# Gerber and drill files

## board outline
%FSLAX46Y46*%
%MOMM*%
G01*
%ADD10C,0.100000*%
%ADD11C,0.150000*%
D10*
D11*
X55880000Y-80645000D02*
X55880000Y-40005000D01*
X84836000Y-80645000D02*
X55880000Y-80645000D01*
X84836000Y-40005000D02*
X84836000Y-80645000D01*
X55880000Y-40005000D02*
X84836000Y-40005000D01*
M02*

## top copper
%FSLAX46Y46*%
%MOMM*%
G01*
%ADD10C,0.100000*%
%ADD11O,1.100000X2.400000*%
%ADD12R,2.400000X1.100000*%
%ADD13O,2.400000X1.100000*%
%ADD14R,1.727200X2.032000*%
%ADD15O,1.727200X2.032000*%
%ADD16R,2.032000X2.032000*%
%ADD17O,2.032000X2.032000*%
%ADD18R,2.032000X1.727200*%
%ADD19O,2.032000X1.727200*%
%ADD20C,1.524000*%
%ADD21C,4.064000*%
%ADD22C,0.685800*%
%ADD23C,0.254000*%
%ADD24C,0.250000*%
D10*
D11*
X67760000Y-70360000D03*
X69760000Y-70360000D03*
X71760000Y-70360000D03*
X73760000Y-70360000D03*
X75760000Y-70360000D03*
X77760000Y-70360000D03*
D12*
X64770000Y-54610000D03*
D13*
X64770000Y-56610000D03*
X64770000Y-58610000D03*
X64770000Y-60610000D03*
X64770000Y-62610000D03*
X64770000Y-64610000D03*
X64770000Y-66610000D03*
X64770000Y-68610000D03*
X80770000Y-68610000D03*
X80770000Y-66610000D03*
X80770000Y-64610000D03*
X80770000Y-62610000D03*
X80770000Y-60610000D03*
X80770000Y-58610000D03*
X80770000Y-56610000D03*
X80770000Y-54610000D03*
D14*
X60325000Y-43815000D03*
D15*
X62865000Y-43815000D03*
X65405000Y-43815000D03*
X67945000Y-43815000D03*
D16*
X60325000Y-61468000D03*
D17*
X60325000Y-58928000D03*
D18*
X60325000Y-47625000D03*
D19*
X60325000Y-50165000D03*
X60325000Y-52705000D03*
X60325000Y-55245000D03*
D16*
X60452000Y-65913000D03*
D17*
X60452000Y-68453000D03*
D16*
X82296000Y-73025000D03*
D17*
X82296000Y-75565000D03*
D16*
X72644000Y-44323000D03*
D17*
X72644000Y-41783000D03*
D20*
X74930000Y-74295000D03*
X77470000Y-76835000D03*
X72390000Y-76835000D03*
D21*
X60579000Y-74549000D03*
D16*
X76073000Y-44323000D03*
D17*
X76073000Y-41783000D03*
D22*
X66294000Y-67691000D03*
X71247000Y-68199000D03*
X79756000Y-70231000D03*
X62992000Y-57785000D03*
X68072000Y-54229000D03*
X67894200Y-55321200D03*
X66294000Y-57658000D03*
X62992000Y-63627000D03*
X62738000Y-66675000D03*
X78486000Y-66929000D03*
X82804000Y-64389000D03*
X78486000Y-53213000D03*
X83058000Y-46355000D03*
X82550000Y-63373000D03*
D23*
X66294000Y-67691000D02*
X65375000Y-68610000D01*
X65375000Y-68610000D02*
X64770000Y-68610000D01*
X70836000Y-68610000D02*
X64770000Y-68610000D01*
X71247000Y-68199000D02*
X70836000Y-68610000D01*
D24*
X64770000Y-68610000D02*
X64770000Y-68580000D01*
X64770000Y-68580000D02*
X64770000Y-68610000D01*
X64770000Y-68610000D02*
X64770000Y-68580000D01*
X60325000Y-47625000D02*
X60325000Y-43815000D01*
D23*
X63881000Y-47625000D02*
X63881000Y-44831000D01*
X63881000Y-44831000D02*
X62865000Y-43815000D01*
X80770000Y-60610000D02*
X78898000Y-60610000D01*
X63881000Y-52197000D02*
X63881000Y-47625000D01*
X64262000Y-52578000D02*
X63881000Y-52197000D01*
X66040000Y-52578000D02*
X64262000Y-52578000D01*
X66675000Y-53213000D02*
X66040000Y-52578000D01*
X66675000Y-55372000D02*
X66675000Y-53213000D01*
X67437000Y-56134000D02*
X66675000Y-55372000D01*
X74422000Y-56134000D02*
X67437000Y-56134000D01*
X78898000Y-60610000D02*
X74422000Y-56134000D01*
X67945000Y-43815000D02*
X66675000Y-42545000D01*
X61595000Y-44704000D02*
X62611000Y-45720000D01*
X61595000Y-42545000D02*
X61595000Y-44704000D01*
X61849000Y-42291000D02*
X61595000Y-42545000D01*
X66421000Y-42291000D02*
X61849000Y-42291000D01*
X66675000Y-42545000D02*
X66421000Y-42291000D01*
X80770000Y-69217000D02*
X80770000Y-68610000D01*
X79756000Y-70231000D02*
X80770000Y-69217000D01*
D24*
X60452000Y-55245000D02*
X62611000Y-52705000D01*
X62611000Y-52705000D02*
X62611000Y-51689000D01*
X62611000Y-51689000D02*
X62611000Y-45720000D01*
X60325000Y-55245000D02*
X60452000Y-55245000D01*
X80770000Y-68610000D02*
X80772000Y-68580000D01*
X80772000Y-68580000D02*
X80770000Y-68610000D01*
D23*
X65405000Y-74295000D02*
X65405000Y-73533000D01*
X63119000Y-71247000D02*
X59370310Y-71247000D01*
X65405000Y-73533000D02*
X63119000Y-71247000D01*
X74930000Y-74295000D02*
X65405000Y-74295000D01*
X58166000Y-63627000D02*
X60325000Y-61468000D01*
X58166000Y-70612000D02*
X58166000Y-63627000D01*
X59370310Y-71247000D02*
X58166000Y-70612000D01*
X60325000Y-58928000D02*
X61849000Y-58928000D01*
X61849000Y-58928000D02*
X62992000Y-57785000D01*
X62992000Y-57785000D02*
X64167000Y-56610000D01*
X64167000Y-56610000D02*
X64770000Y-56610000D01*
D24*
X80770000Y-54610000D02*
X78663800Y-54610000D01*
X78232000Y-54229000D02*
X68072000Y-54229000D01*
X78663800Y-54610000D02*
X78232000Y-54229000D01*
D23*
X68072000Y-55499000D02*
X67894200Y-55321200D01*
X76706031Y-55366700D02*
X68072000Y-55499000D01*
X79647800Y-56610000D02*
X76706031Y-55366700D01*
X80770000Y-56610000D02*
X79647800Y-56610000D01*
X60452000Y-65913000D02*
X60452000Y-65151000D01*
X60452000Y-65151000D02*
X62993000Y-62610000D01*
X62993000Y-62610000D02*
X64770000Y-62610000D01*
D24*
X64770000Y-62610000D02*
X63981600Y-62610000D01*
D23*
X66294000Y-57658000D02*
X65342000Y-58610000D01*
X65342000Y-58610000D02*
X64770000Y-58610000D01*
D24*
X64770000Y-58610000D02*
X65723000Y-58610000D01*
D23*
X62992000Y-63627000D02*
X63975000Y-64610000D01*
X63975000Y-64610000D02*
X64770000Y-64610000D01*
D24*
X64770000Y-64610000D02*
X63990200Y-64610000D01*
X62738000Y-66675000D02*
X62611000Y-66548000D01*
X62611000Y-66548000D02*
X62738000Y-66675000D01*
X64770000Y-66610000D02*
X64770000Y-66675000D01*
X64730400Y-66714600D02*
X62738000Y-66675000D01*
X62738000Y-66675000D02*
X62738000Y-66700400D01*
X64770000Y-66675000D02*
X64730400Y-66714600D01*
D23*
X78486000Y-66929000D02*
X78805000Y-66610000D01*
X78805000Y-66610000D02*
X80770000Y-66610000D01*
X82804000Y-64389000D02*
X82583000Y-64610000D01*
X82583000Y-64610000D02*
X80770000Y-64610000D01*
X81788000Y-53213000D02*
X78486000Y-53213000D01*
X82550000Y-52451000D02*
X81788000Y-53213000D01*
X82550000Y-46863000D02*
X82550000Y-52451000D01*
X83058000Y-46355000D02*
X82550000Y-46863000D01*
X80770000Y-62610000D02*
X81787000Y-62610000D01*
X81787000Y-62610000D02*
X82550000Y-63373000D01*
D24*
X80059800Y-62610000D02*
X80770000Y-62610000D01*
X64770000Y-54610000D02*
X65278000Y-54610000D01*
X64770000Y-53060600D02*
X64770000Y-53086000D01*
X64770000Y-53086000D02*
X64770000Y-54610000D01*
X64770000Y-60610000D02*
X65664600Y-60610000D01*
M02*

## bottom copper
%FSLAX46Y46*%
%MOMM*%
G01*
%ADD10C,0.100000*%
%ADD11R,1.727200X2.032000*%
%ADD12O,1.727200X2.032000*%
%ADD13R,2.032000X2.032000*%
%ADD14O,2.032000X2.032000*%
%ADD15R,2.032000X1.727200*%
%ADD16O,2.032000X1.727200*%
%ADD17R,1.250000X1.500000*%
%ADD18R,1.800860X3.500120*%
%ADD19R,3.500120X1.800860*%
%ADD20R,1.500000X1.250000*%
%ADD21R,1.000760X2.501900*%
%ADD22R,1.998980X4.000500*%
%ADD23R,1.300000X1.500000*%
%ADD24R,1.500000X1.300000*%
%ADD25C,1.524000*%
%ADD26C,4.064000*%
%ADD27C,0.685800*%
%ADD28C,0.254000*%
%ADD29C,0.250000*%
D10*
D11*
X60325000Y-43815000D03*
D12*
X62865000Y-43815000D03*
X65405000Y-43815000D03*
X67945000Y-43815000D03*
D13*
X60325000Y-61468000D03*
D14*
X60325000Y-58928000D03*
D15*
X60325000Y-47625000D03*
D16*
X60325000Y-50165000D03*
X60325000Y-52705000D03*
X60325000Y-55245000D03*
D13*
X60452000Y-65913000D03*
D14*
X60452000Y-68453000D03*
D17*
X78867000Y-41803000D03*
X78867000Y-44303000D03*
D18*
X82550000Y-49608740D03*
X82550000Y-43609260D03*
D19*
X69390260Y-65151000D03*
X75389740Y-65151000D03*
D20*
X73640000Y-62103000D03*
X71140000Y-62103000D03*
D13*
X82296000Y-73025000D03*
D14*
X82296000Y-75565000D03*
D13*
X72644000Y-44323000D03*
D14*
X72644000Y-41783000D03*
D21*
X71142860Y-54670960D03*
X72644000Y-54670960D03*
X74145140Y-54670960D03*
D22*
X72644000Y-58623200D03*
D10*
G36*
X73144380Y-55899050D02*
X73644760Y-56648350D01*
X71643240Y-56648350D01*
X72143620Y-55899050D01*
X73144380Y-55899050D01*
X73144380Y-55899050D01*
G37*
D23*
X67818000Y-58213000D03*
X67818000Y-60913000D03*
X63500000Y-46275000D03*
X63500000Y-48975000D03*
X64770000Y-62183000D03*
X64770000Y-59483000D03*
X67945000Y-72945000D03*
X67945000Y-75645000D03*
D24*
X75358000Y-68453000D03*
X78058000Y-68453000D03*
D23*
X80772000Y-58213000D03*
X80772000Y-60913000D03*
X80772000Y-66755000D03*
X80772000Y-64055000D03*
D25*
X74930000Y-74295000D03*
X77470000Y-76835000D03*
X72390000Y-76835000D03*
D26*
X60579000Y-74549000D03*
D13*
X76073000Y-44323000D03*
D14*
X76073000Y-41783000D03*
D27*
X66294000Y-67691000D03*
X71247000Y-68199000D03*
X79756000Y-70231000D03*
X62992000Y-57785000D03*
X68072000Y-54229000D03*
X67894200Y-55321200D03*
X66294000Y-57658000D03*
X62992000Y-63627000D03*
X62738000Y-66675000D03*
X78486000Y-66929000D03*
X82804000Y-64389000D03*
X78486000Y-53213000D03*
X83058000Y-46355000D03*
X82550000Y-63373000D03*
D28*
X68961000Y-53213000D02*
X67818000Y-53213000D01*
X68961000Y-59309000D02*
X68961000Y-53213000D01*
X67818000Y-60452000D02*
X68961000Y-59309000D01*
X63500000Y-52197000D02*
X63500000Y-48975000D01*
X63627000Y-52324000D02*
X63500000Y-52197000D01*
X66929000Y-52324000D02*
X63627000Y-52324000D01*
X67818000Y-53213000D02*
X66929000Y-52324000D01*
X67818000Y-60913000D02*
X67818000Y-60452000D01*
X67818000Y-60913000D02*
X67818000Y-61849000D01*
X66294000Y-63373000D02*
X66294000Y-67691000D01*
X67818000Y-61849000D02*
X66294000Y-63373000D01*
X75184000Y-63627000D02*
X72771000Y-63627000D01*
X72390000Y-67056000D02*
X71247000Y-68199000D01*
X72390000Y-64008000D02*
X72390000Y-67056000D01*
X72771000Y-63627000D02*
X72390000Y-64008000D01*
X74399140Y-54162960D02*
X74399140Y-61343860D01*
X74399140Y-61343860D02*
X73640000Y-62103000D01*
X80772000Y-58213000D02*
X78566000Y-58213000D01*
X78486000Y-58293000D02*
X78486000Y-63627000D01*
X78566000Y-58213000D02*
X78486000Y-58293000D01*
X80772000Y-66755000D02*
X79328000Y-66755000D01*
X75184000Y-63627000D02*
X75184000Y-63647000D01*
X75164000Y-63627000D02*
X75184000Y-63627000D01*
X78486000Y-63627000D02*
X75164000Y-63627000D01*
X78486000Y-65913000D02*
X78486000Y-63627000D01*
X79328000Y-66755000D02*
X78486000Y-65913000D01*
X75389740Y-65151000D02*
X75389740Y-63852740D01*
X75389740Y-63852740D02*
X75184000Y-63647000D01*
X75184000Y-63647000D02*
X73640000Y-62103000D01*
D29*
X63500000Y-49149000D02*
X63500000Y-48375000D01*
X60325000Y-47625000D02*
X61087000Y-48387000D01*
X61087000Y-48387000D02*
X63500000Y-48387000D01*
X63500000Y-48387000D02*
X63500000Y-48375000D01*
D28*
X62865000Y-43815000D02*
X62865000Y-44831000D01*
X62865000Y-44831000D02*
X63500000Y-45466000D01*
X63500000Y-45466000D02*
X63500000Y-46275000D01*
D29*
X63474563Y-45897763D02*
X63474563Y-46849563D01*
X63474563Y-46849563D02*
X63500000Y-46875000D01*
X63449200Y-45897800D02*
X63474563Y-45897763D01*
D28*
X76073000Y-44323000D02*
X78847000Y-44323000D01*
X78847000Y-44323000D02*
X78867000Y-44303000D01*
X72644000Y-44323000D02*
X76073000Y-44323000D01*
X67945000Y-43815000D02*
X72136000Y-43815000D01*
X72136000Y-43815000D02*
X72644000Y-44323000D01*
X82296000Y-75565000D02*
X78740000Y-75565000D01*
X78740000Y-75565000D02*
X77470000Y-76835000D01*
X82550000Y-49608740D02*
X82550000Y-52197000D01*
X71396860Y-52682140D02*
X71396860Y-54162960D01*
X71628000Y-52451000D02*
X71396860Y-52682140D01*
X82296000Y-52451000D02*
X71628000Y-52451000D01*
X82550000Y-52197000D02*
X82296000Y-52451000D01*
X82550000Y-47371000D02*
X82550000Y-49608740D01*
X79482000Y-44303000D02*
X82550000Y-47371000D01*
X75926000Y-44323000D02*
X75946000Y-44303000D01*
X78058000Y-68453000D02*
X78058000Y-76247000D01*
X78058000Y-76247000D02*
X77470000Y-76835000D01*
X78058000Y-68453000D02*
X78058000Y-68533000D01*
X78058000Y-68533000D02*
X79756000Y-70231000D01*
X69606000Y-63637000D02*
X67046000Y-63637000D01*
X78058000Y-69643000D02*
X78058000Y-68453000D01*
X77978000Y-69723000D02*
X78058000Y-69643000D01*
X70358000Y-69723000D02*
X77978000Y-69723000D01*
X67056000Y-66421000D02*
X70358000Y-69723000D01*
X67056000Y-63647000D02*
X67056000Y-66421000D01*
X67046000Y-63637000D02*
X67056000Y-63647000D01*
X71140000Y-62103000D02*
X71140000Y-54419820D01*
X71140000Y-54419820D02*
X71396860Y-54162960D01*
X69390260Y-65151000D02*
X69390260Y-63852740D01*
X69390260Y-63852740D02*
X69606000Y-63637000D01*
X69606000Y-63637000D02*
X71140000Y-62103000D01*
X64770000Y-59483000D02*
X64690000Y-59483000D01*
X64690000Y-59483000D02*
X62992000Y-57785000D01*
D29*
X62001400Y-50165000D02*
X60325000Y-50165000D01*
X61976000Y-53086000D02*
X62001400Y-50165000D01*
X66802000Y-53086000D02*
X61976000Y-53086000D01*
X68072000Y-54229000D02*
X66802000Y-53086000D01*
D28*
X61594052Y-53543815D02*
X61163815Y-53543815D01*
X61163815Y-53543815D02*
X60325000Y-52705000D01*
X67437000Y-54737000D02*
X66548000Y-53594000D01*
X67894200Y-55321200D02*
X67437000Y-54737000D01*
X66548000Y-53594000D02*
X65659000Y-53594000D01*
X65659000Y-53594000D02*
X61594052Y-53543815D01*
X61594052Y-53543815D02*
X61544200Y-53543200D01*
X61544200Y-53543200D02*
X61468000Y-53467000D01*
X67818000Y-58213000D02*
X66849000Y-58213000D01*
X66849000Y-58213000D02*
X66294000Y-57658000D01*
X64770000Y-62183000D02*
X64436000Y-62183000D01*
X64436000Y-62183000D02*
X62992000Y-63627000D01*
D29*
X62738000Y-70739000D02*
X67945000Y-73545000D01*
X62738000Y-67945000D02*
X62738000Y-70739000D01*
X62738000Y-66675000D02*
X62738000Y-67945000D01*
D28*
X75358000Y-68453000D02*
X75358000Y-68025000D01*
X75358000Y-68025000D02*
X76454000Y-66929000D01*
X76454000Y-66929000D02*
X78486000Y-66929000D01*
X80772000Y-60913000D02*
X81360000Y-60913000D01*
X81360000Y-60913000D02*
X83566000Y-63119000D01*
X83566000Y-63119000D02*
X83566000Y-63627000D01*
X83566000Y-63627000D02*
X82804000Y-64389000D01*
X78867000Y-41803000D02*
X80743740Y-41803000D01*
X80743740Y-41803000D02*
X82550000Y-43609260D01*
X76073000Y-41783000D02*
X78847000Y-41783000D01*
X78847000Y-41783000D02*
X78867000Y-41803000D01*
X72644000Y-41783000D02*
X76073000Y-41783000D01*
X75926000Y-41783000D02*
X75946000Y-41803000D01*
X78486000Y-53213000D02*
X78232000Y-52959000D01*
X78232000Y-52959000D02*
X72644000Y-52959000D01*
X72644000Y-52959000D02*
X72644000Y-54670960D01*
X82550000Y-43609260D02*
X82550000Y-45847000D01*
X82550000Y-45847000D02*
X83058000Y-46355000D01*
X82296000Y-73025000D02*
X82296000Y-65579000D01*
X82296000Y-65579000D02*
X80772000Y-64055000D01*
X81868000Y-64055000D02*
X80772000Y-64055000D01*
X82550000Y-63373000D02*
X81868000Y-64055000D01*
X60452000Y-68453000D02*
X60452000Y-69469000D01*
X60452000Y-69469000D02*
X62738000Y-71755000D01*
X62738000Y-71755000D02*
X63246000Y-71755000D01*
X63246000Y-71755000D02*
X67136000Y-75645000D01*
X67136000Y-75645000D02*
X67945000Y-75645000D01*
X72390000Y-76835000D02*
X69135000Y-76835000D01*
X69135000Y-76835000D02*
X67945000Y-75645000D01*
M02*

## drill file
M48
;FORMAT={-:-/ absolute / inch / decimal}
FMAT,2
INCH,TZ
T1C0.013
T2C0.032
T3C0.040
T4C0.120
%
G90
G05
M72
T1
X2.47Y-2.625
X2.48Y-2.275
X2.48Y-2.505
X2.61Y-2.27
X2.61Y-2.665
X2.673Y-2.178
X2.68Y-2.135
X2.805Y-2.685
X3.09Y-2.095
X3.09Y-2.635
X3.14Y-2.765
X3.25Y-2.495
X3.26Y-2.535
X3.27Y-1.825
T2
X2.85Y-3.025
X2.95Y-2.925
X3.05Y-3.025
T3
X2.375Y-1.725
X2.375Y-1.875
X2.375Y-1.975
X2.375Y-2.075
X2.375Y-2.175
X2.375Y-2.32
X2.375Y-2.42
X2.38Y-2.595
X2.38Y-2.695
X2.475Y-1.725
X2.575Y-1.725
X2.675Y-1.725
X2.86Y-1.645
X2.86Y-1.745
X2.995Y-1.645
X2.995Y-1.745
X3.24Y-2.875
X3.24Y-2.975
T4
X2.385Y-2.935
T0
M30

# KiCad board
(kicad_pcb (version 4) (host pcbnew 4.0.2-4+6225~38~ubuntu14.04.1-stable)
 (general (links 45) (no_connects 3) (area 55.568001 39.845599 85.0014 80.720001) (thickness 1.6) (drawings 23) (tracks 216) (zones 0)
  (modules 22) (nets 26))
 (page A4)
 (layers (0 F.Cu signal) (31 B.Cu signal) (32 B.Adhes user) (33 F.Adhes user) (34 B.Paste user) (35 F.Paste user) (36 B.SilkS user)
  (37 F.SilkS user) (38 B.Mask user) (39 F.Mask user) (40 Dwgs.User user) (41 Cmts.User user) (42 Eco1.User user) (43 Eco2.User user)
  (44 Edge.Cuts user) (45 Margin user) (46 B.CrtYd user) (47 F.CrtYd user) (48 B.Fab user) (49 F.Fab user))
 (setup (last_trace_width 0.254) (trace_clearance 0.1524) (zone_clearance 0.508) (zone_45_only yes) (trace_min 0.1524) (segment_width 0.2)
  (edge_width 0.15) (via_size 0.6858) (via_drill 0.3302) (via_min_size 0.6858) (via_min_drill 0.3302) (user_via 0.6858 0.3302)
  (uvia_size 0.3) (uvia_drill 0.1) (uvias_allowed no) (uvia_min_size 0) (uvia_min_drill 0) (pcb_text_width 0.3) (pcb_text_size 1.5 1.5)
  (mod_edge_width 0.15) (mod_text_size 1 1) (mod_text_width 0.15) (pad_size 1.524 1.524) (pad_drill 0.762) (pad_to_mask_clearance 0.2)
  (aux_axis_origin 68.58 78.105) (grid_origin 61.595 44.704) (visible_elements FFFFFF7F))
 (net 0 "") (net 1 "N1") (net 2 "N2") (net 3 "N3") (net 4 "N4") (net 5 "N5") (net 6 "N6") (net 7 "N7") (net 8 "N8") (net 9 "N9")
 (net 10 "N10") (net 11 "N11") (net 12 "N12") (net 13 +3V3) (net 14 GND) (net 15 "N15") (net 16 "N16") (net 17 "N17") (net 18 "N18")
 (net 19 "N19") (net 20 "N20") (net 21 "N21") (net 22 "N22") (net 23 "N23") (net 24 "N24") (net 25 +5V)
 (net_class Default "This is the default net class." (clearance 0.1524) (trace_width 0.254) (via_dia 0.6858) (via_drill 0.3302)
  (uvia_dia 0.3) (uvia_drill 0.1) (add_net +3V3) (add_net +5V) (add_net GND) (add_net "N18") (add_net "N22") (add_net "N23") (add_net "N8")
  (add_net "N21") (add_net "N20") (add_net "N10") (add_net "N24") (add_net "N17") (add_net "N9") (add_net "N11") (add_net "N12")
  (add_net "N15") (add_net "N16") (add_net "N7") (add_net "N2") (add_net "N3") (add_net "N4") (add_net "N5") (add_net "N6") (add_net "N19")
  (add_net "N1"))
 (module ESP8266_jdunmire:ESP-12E (layer F.Cu) (at 64.77 54.61)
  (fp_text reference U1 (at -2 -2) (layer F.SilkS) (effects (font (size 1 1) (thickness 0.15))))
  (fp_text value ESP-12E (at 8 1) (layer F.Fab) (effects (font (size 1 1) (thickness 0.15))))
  (pad 9 smd oval (at 2.99 15.75 90) (size 2.4 1.1) (layers F.Cu F.Paste F.Mask) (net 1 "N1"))
  (pad 10 smd oval (at 4.99 15.75 90) (size 2.4 1.1) (layers F.Cu F.Paste F.Mask) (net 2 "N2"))
  (pad 11 smd oval (at 6.99 15.75 90) (size 2.4 1.1) (layers F.Cu F.Paste F.Mask) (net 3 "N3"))
  (pad 12 smd oval (at 8.99 15.75 90) (size 2.4 1.1) (layers F.Cu F.Paste F.Mask) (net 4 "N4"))
  (pad 13 smd oval (at 10.99 15.75 90) (size 2.4 1.1) (layers F.Cu F.Paste F.Mask) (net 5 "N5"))
  (pad 14 smd oval (at 12.99 15.75 90) (size 2.4 1.1) (layers F.Cu F.Paste F.Mask) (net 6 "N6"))
  (pad 1 smd rect (at 0 0) (size 2.4 1.1) (layers F.Cu F.Paste F.Mask) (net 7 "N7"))
  (pad 2 smd oval (at 0 2) (size 2.4 1.1) (layers F.Cu F.Paste F.Mask) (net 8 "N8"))
  (pad 3 smd oval (at 0 4) (size 2.4 1.1) (layers F.Cu F.Paste F.Mask) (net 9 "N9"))
  (pad 4 smd oval (at 0 6) (size 2.4 1.1) (layers F.Cu F.Paste F.Mask) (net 7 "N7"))
  (pad 5 smd oval (at 0 8) (size 2.4 1.1) (layers F.Cu F.Paste F.Mask) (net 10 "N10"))
  (pad 6 smd oval (at 0 10) (size 2.4 1.1) (layers F.Cu F.Paste F.Mask) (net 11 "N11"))
  (pad 7 smd oval (at 0 12) (size 2.4 1.1) (layers F.Cu F.Paste F.Mask) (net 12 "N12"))
  (pad 8 smd oval (at 0 14) (size 2.4 1.1) (layers F.Cu F.Paste F.Mask) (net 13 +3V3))
  (pad 15 smd oval (at 16 14) (size 2.4 1.1) (layers F.Cu F.Paste F.Mask) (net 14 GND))
  (pad 16 smd oval (at 16 12) (size 2.4 1.1) (layers F.Cu F.Paste F.Mask) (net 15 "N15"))
  (pad 17 smd oval (at 16 10) (size 2.4 1.1) (layers F.Cu F.Paste F.Mask) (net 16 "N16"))
  (pad 18 smd oval (at 16 8) (size 2.4 1.1) (layers F.Cu F.Paste F.Mask) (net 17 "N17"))
  (pad 19 smd oval (at 16 6) (size 2.4 1.1) (layers F.Cu F.Paste F.Mask) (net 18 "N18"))
  (pad 20 smd oval (at 16 4) (size 2.4 1.1) (layers F.Cu F.Paste F.Mask) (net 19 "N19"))
  (pad 21 smd oval (at 16 2) (size 2.4 1.1) (layers F.Cu F.Paste F.Mask) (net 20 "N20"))
  (pad 22 smd oval (at 16 0) (size 2.4 1.1) (layers F.Cu F.Paste F.Mask) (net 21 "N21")))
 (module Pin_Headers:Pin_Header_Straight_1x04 (layer F.Cu) (at 60.325 43.815 90)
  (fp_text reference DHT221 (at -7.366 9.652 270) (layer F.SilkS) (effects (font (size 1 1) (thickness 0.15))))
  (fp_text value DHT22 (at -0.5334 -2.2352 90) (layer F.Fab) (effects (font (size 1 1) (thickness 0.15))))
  (pad 1 thru_hole rect (at 0 0 90) (size 2.032 1.7272) (drill 1.016) (layers *.Cu *.Mask F.SilkS) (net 13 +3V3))
  (pad 2 thru_hole oval (at 0 2.54 90) (size 2.032 1.7272) (drill 1.016) (layers *.Cu *.Mask F.SilkS) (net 18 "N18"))
  (pad 3 thru_hole oval (at 0 5.08 90) (size 2.032 1.7272) (drill 1.016) (layers *.Cu *.Mask F.SilkS) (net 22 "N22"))
  (pad 4 thru_hole oval (at 0 7.62 90) (size 2.032 1.7272) (drill 1.016) (layers *.Cu *.Mask F.SilkS) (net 14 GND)))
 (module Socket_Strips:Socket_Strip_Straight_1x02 (layer F.Cu) (at 60.325 61.468 90)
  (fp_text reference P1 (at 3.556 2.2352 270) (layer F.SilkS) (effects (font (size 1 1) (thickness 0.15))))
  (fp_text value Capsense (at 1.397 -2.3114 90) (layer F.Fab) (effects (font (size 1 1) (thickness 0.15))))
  (pad 1 thru_hole rect (at 0 0 90) (size 2.032 2.032) (drill 1.016) (layers *.Cu *.Mask F.SilkS) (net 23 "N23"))
  (pad 2 thru_hole oval (at 2.54 0 90) (size 2.032 2.032) (drill 1.016) (layers *.Cu *.Mask F.SilkS) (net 8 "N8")))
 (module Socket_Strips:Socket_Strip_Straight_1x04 (layer F.Cu) (at 60.325 47.625 270)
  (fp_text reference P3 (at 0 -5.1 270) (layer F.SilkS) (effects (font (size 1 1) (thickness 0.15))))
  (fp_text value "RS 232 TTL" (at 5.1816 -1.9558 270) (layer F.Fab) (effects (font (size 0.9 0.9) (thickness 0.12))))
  (pad 1 thru_hole rect (at 0 0 270) (size 1.7272 2.032) (drill 1.016) (layers *.Cu *.Mask F.SilkS) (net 13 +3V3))
  (pad 2 thru_hole oval (at 2.54 0 270) (size 1.7272 2.032) (drill 1.016) (layers *.Cu *.Mask F.SilkS) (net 21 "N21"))
  (pad 3 thru_hole oval (at 5.08 0 270) (size 1.7272 2.032) (drill 1.016) (layers *.Cu *.Mask F.SilkS) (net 20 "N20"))
  (pad 4 thru_hole oval (at 7.62 0 270) (size 1.7272 2.032) (drill 1.016) (layers *.Cu *.Mask F.SilkS) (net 14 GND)))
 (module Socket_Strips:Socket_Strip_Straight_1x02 (layer F.Cu) (at 60.452 65.913 270)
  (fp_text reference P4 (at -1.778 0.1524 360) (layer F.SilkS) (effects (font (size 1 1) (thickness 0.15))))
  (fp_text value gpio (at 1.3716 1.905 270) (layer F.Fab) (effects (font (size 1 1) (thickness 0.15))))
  (pad 1 thru_hole rect (at 0 0 270) (size 2.032 2.032) (drill 1.016) (layers *.Cu *.Mask F.SilkS) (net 10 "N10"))
  (pad 2 thru_hole oval (at 2.54 0 270) (size 2.032 2.032) (drill 1.016) (layers *.Cu *.Mask F.SilkS) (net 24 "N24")))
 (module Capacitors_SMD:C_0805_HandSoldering (layer B.Cu) (at 78.867 43.053 270)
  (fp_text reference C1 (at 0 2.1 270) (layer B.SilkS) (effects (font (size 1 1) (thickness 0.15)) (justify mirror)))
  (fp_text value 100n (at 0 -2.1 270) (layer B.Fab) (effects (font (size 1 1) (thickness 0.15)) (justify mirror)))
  (pad 1 smd rect (at -1.25 0 270) (size 1.5 1.25) (layers B.Cu B.Paste B.Mask) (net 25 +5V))
  (pad 2 smd rect (at 1.25 0 270) (size 1.5 1.25) (layers B.Cu B.Paste B.Mask) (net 14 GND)))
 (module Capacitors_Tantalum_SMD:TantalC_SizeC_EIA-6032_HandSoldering (layer B.Cu) (at 82.55 46.609 270)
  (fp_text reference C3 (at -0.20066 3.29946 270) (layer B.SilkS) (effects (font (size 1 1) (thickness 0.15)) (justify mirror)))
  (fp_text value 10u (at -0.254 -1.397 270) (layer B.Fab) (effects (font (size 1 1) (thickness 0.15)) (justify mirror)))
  (pad 2 smd rect (at 2.99974 0 270) (size 3.50012 1.80086) (layers B.Cu B.Paste B.Mask) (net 14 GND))
  (pad 1 smd rect (at -2.99974 0 270) (size 3.50012 1.80086) (layers B.Cu B.Paste B.Mask) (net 25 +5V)))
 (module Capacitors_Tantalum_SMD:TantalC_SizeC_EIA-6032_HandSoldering (layer B.Cu) (at 72.39 65.151 180)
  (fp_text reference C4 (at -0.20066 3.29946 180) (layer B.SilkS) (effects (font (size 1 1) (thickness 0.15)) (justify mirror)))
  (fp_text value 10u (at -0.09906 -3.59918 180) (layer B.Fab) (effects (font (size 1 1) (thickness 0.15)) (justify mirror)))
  (pad 2 smd rect (at 2.99974 0 180) (size 3.50012 1.80086) (layers B.Cu B.Paste B.Mask) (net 14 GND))
  (pad 1 smd rect (at -2.99974 0 180) (size 3.50012 1.80086) (layers B.Cu B.Paste B.Mask) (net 13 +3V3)))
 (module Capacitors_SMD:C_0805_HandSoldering (layer B.Cu) (at 72.39 62.103 180)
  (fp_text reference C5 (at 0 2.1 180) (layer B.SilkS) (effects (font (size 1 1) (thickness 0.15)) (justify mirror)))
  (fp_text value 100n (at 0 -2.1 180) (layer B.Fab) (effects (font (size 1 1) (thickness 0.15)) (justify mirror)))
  (pad 1 smd rect (at -1.25 0 180) (size 1.5 1.25) (layers B.Cu B.Paste B.Mask) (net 13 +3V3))
  (pad 2 smd rect (at 1.25 0 180) (size 1.5 1.25) (layers B.Cu B.Paste B.Mask) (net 14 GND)))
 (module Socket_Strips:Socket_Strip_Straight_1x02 (layer F.Cu) (at 82.296 73.025 270)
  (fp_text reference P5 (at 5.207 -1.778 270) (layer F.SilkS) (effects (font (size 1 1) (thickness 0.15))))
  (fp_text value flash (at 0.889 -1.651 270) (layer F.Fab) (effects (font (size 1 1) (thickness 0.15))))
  (pad 1 thru_hole rect (at 0 0 270) (size 2.032 2.032) (drill 1.016) (layers *.Cu *.Mask F.SilkS) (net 17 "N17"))
  (pad 2 thru_hole oval (at 2.54 0 270) (size 2.032 2.032) (drill 1.016) (layers *.Cu *.Mask F.SilkS) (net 14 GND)))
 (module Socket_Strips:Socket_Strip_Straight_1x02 (layer F.Cu) (at 72.644 44.323 90)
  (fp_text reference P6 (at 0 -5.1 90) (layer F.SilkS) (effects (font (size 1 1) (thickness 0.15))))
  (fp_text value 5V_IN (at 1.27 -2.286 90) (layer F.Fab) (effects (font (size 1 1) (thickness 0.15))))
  (pad 1 thru_hole rect (at 0 0 90) (size 2.032 2.032) (drill 1.016) (layers *.Cu *.Mask F.SilkS) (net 14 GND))
  (pad 2 thru_hole oval (at 2.54 0 90) (size 2.032 2.032) (drill 1.016) (layers *.Cu *.Mask F.SilkS) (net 25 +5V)))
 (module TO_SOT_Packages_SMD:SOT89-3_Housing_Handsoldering (layer B.Cu) (at 72.644 57.023)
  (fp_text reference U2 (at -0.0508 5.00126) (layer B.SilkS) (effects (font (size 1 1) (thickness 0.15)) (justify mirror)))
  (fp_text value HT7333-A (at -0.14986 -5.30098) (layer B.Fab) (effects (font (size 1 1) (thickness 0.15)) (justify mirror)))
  (pad 1 smd rect (at -1.50114 -2.35204) (size 1.00076 2.5019) (layers B.Cu B.Paste B.Mask) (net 14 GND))
  (pad 2 smd rect (at 0 -2.35204) (size 1.00076 2.5019) (layers B.Cu B.Paste B.Mask) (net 25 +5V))
  (pad 3 smd rect (at 1.50114 -2.35204) (size 1.00076 2.5019) (layers B.Cu B.Paste B.Mask) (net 13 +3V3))
  (pad 2 smd rect (at 0 1.6002) (size 1.99898 4.0005) (layers B.Cu B.Paste B.Mask) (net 25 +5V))
  (pad 2 smd trapezoid (at 0 -0.7493 180) (size 1.50114 0.7493) (rect_delta 0 -0.50038) (layers B.Cu B.Paste B.Mask) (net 25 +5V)))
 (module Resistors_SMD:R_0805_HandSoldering (layer B.Cu) (at 67.818 59.563 270)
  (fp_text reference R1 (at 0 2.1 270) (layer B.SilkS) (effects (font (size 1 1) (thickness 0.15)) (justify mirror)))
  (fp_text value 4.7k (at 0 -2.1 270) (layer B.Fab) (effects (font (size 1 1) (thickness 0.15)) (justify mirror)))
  (pad 1 smd rect (at -1.35 0 270) (size 1.5 1.3) (layers B.Cu B.Paste B.Mask) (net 9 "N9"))
  (pad 2 smd rect (at 1.35 0 270) (size 1.5 1.3) (layers B.Cu B.Paste B.Mask) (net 13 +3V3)))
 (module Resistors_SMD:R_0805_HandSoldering (layer B.Cu) (at 63.5 47.625 270)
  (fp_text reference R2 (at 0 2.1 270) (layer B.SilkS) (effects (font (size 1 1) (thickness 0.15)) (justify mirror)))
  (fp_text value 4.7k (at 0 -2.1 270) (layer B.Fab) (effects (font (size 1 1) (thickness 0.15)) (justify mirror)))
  (pad 1 smd rect (at -1.35 0 270) (size 1.5 1.3) (layers B.Cu B.Paste B.Mask) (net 18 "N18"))
  (pad 2 smd rect (at 1.35 0 270) (size 1.5 1.3) (layers B.Cu B.Paste B.Mask) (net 13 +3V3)))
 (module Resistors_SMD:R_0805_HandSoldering (layer B.Cu) (at 64.77 60.833 90)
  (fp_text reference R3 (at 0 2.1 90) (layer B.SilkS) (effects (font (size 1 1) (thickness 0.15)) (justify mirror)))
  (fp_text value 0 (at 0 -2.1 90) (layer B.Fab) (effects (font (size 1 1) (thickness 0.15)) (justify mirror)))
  (pad 1 smd rect (at -1.35 0 90) (size 1.5 1.3) (layers B.Cu B.Paste B.Mask) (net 11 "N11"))
  (pad 2 smd rect (at 1.35 0 90) (size 1.5 1.3) (layers B.Cu B.Paste B.Mask) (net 8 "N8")))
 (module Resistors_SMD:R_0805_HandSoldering (layer B.Cu) (at 67.945 74.295 270)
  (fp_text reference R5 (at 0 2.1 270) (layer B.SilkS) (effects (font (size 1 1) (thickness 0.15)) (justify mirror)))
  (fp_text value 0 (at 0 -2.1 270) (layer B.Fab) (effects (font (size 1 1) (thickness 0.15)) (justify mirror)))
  (pad 1 smd rect (at -1.35 0 270) (size 1.5 1.3) (layers B.Cu B.Paste B.Mask) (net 12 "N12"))
  (pad 2 smd rect (at 1.35 0 270) (size 1.5 1.3) (layers B.Cu B.Paste B.Mask) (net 24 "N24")))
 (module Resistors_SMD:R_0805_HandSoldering (layer B.Cu) (at 76.708 68.453)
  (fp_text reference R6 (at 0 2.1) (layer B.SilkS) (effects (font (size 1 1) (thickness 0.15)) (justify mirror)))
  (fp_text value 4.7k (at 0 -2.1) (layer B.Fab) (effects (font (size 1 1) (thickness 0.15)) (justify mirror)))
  (pad 1 smd rect (at -1.35 0) (size 1.5 1.3) (layers B.Cu B.Paste B.Mask) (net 15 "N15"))
  (pad 2 smd rect (at 1.35 0) (size 1.5 1.3) (layers B.Cu B.Paste B.Mask) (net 14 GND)))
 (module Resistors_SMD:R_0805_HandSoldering (layer B.Cu) (at 80.772 59.563 270)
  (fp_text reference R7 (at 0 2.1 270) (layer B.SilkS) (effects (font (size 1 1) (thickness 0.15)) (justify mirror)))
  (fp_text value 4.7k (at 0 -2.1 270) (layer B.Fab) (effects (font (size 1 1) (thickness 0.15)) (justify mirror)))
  (pad 1 smd rect (at -1.35 0 270) (size 1.5 1.3) (layers B.Cu B.Paste B.Mask) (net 13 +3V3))
  (pad 2 smd rect (at 1.35 0 270) (size 1.5 1.3) (layers B.Cu B.Paste B.Mask) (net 16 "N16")))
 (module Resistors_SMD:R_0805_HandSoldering (layer B.Cu) (at 80.772 65.405 90)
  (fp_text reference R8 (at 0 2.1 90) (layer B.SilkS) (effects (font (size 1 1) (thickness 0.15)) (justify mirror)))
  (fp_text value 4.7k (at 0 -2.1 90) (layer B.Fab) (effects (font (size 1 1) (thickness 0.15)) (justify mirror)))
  (pad 1 smd rect (at -1.35 0 90) (size 1.5 1.3) (layers B.Cu B.Paste B.Mask) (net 13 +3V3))
  (pad 2 smd rect (at 1.35 0 90) (size 1.5 1.3) (layers B.Cu B.Paste B.Mask) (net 17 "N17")))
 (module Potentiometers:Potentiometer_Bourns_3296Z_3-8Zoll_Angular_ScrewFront (layer F.Cu) (at 72.39 76.835 270)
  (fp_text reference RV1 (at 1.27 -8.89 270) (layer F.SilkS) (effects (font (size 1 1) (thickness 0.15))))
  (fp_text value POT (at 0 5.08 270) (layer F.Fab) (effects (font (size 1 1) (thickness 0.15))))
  (pad 2 thru_hole circle (at -2.54 -2.54 270) (size 1.524 1.524) (drill 0.8128) (layers *.Cu *.Mask F.SilkS) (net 23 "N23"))
  (pad 3 thru_hole circle (at 0 -5.08 270) (size 1.524 1.524) (drill 0.8128) (layers *.Cu *.Mask F.SilkS) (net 14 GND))
  (pad 1 thru_hole circle (at 0 0 270) (size 1.524 1.524) (drill 0.8128) (layers *.Cu *.Mask F.SilkS) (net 24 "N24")))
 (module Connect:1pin (layer F.Cu) (at 60.579 74.549)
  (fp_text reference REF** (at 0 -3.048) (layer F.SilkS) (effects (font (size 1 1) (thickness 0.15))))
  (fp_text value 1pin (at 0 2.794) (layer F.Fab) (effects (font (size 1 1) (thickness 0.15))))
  (pad 1 thru_hole circle (at 0 0) (size 4.064 4.064) (drill 3.048) (layers *.Cu *.Mask F.SilkS)))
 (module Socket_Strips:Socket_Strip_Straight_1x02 (layer F.Cu) (at 76.073 44.323 90)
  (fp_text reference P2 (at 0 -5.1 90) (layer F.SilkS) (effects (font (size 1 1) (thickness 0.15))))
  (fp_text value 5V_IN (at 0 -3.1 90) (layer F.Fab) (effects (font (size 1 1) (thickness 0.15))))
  (pad 1 thru_hole rect (at 0 0 90) (size 2.032 2.032) (drill 1.016) (layers *.Cu *.Mask F.SilkS) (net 14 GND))
  (pad 2 thru_hole oval (at 2.54 0 90) (size 2.032 2.032) (drill 1.016) (layers *.Cu *.Mask F.SilkS) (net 25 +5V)))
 (gr_line (start 55.88 80.645) (end 55.88 40.005) (angle 90) (layer Edge.Cuts) (width 0.15))
 (gr_line (start 84.836 80.645) (end 55.88 80.645) (angle 90) (layer Edge.Cuts) (width 0.15))
 (gr_line (start 84.836 40.005) (end 84.836 80.645) (angle 90) (layer Edge.Cuts) (width 0.15))
 (gr_line (start 55.88 40.005) (end 84.836 40.005) (angle 90) (layer Edge.Cuts) (width 0.15))
 (segment (start 68.961 53.213) (end 67.818 53.213) (width 0.254) (layer B.Cu) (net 13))
 (segment (start 68.961 59.309) (end 68.961 53.213) (width 0.254) (layer B.Cu) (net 13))
 (segment (start 67.818 60.452) (end 68.961 59.309) (width 0.254) (layer B.Cu) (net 13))
 (segment (start 63.5 52.197) (end 63.5 48.975) (width 0.254) (layer B.Cu) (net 13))
 (segment (start 63.627 52.324) (end 63.5 52.197) (width 0.254) (layer B.Cu) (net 13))
 (segment (start 66.929 52.324) (end 63.627 52.324) (width 0.254) (layer B.Cu) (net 13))
 (segment (start 67.818 53.213) (end 66.929 52.324) (width 0.254) (layer B.Cu) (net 13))
 (segment (start 67.818 60.913) (end 67.818 60.452) (width 0.254) (layer B.Cu) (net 13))
 (segment (start 67.818 60.913) (end 67.818 61.849) (width 0.254) (layer B.Cu) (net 13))
 (segment (start 66.294 67.691) (end 65.375 68.61) (width 0.254) (layer F.Cu) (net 13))
 (via (at 66.294 67.691) (size 0.6858) (drill 0.3302) (layers F.Cu B.Cu) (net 13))
 (segment (start 66.294 63.373) (end 66.294 67.691) (width 0.254) (layer B.Cu) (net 13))
 (segment (start 67.818 61.849) (end 66.294 63.373) (width 0.254) (layer B.Cu) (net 13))
 (segment (start 65.375 68.61) (end 64.77 68.61) (width 0.254) (layer F.Cu) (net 13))
 (segment (start 75.184 63.627) (end 72.771 63.627) (width 0.254) (layer B.Cu) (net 13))
 (segment (start 70.836 68.61) (end 64.77 68.61) (width 0.254) (layer F.Cu) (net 13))
 (segment (start 71.247 68.199) (end 70.836 68.61) (width 0.254) (layer F.Cu) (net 13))
 (via (at 71.247 68.199) (size 0.6858) (drill 0.3302) (layers F.Cu B.Cu) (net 13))
 (segment (start 72.39 67.056) (end 71.247 68.199) (width 0.254) (layer B.Cu) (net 13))
 (segment (start 72.39 64.008) (end 72.39 67.056) (width 0.254) (layer B.Cu) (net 13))
 (segment (start 72.771 63.627) (end 72.39 64.008) (width 0.254) (layer B.Cu) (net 13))
 (segment (start 74.39914 54.16296) (end 74.39914 61.34386) (width 0.254) (layer B.Cu) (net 13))
 (segment (start 74.39914 61.34386) (end 73.64 62.103) (width 0.254) (layer B.Cu) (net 13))
 (segment (start 80.772 58.213) (end 78.566 58.213) (width 0.254) (layer B.Cu) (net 13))
 (segment (start 78.486 58.293) (end 78.486 63.627) (width 0.254) (layer B.Cu) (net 13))
 (segment (start 78.566 58.213) (end 78.486 58.293) (width 0.254) (layer B.Cu) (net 13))
 (segment (start 80.772 66.755) (end 79.328 66.755) (width 0.254) (layer B.Cu) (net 13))
 (segment (start 75.184 63.627) (end 75.184 63.647) (width 0.254) (layer B.Cu) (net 13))
 (segment (start 75.164 63.627) (end 75.184 63.627) (width 0.254) (layer B.Cu) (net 13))
 (segment (start 78.486 63.627) (end 75.164 63.627) (width 0.254) (layer B.Cu) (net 13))
 (segment (start 78.486 65.913) (end 78.486 63.627) (width 0.254) (layer B.Cu) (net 13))
 (segment (start 79.328 66.755) (end 78.486 65.913) (width 0.254) (layer B.Cu) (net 13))
 (segment (start 75.38974 65.151) (end 75.38974 63.85274) (width 0.254) (layer B.Cu) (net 13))
 (segment (start 75.38974 63.85274) (end 75.184 63.647) (width 0.254) (layer B.Cu) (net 13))
 (segment (start 75.184 63.647) (end 73.64 62.103) (width 0.254) (layer B.Cu) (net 13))
 (segment (start 63.5 49.149) (end 63.5 48.375) (width 0.25) (layer B.Cu) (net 13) (status 80000))
 (segment (start 64.77 68.61) (end 64.77 68.58) (width 0.25) (layer F.Cu) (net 13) (status 80000))
 (segment (start 64.77 68.58) (end 64.77 68.61) (width 0.25) (layer F.Cu) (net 13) (status 80000))
 (segment (start 64.77 68.61) (end 64.77 68.58) (width 0.25) (layer F.Cu) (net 13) (status 80000))
 (segment (start 60.325 47.625) (end 61.087 48.387) (width 0.25) (layer B.Cu) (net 13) (status 80000))
 (segment (start 61.087 48.387) (end 63.5 48.387) (width 0.25) (layer B.Cu) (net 13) (status 80000))
 (segment (start 63.5 48.387) (end 63.5 48.375) (width 0.25) (layer B.Cu) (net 13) (status 80000))
 (segment (start 60.325 47.625) (end 60.325 43.815) (width 0.25) (layer F.Cu) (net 13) (status 80000))
 (segment (start 62.865 43.815) (end 62.865 44.831) (width 0.254) (layer B.Cu) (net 18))
 (segment (start 62.865 44.831) (end 63.5 45.466) (width 0.254) (layer B.Cu) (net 18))
 (segment (start 63.5 45.466) (end 63.5 46.275) (width 0.254) (layer B.Cu) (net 18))
 (segment (start 63.881 47.625) (end 63.881 44.831) (width 0.254) (layer F.Cu) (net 18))
 (segment (start 63.881 44.831) (end 62.865 43.815) (width 0.254) (layer F.Cu) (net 18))
 (segment (start 80.77 60.61) (end 78.898 60.61) (width 0.254) (layer F.Cu) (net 18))
 (segment (start 63.881 52.197) (end 63.881 47.625) (width 0.254) (layer F.Cu) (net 18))
 (segment (start 64.262 52.578) (end 63.881 52.197) (width 0.254) (layer F.Cu) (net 18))
 (segment (start 66.04 52.578) (end 64.262 52.578) (width 0.254) (layer F.Cu) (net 18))
 (segment (start 66.675 53.213) (end 66.04 52.578) (width 0.254) (layer F.Cu) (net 18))
 (segment (start 66.675 55.372) (end 66.675 53.213) (width 0.254) (layer F.Cu) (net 18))
 (segment (start 67.437 56.134) (end 66.675 55.372) (width 0.254) (layer F.Cu) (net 18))
 (segment (start 74.422 56.134) (end 67.437 56.134) (width 0.254) (layer F.Cu) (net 18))
 (segment (start 78.898 60.61) (end 74.422 56.134) (width 0.254) (layer F.Cu) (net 18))
 (segment (start 63.474563 45.897763) (end 63.474563 46.849563) (width 0.25) (layer B.Cu) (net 18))
 (segment (start 63.474563 46.849563) (end 63.5 46.875) (width 0.25) (layer B.Cu) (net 18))
 (segment (start 63.4492 45.8978) (end 63.474563 45.897763) (width 0.25) (layer B.Cu) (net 18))
 (segment (start 76.073 44.323) (end 78.847 44.323) (width 0.254) (layer B.Cu) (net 14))
 (segment (start 78.847 44.323) (end 78.867 44.303) (width 0.254) (layer B.Cu) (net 14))
 (segment (start 72.644 44.323) (end 76.073 44.323) (width 0.254) (layer B.Cu) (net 14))
 (segment (start 67.945 43.815) (end 66.675 42.545) (width 0.254) (layer F.Cu) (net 14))
 (segment (start 61.595 44.704) (end 62.611 45.72) (width 0.254) (layer F.Cu) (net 14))
 (segment (start 61.595 42.545) (end 61.595 44.704) (width 0.254) (layer F.Cu) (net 14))
 (segment (start 61.849 42.291) (end 61.595 42.545) (width 0.254) (layer F.Cu) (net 14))
 (segment (start 66.421 42.291) (end 61.849 42.291) (width 0.254) (layer F.Cu) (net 14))
 (segment (start 66.675 42.545) (end 66.421 42.291) (width 0.254) (layer F.Cu) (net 14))
 (segment (start 67.945 43.815) (end 72.136 43.815) (width 0.254) (layer B.Cu) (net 14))
 (segment (start 72.136 43.815) (end 72.644 44.323) (width 0.254) (layer B.Cu) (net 14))
 (segment (start 82.296 75.565) (end 78.74 75.565) (width 0.254) (layer B.Cu) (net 14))
 (segment (start 78.74 75.565) (end 77.47 76.835) (width 0.254) (layer B.Cu) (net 14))
 (segment (start 82.55 49.60874) (end 82.55 52.197) (width 0.254) (layer B.Cu) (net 14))
 (segment (start 71.39686 52.68214) (end 71.39686 54.16296) (width 0.254) (layer B.Cu) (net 14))
 (segment (start 71.628 52.451) (end 71.39686 52.68214) (width 0.254) (layer B.Cu) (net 14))
 (segment (start 82.296 52.451) (end 71.628 52.451) (width 0.254) (layer B.Cu) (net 14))
 (segment (start 82.55 52.197) (end 82.296 52.451) (width 0.254) (layer B.Cu) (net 14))
 (segment (start 82.55 47.371) (end 82.55 49.60874) (width 0.254) (layer B.Cu) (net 14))
 (segment (start 79.482 44.303) (end 82.55 47.371) (width 0.254) (layer B.Cu) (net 14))
 (segment (start 75.926 44.323) (end 75.946 44.303) (width 0.254) (layer B.Cu) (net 14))
 (segment (start 78.058 68.453) (end 78.058 76.247) (width 0.254) (layer B.Cu) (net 14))
 (segment (start 78.058 76.247) (end 77.47 76.835) (width 0.254) (layer B.Cu) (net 14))
 (segment (start 78.058 68.453) (end 78.058 68.533) (width 0.254) (layer B.Cu) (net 14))
 (segment (start 78.058 68.533) (end 79.756 70.231) (width 0.254) (layer B.Cu) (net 14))
 (segment (start 80.77 69.217) (end 80.77 68.61) (width 0.254) (layer F.Cu) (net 14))
 (segment (start 79.756 70.231) (end 80.77 69.217) (width 0.254) (layer F.Cu) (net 14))
 (via (at 79.756 70.231) (size 0.6858) (drill 0.3302) (layers F.Cu B.Cu) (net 14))
 (segment (start 69.606 63.637) (end 67.046 63.637) (width 0.254) (layer B.Cu) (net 14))
 (segment (start 78.058 69.643) (end 78.058 68.453) (width 0.254) (layer B.Cu) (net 14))
 (segment (start 77.978 69.723) (end 78.058 69.643) (width 0.254) (layer B.Cu) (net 14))
 (segment (start 70.358 69.723) (end 77.978 69.723) (width 0.254) (layer B.Cu) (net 14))
 (segment (start 67.056 66.421) (end 70.358 69.723) (width 0.254) (layer B.Cu) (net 14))
 (segment (start 67.056 63.647) (end 67.056 66.421) (width 0.254) (layer B.Cu) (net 14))
 (segment (start 67.046 63.637) (end 67.056 63.647) (width 0.254) (layer B.Cu) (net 14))
 (segment (start 71.14 62.103) (end 71.14 54.41982) (width 0.254) (layer B.Cu) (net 14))
 (segment (start 71.14 54.41982) (end 71.39686 54.16296) (width 0.254) (layer B.Cu) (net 14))
 (segment (start 69.39026 65.151) (end 69.39026 63.85274) (width 0.254) (layer B.Cu) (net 14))
 (segment (start 69.39026 63.85274) (end 69.606 63.637) (width 0.254) (layer B.Cu) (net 14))
 (segment (start 69.606 63.637) (end 71.14 62.103) (width 0.254) (layer B.Cu) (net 14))
 (segment (start 60.452 55.245) (end 62.611 52.705) (width 0.25) (layer F.Cu) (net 14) (status 80000))
 (segment (start 62.611 52.705) (end 62.611 51.689) (width 0.25) (layer F.Cu) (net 14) (status 80000))
 (segment (start 62.611 51.689) (end 62.611 45.72) (width 0.25) (layer F.Cu) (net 14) (status 80000))
 (segment (start 60.325 55.245) (end 60.452 55.245) (width 0.25) (layer F.Cu) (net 14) (status 80000))
 (segment (start 80.77 68.61) (end 80.772 68.58) (width 0.25) (layer F.Cu) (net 14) (status 80000))
 (segment (start 80.772 68.58) (end 80.77 68.61) (width 0.25) (layer F.Cu) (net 14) (status 80000))
 (segment (start 65.405 74.295) (end 65.405 73.533) (width 0.254) (layer F.Cu) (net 23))
 (segment (start 63.119 71.247) (end 59.37031 71.247) (width 0.254) (layer F.Cu) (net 23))
 (segment (start 65.405 73.533) (end 63.119 71.247) (width 0.254) (layer F.Cu) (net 23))
 (segment (start 74.93 74.295) (end 65.405 74.295) (width 0.254) (layer F.Cu) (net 23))
 (segment (start 58.166 63.627) (end 60.325 61.468) (width 0.254) (layer F.Cu) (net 23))
 (segment (start 58.166 70.612) (end 58.166 63.627) (width 0.254) (layer F.Cu) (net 23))
 (segment (start 59.37031 71.247) (end 58.166 70.612) (width 0.254) (layer F.Cu) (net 23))
 (segment (start 60.325 58.928) (end 61.849 58.928) (width 0.254) (layer F.Cu) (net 8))
 (segment (start 61.849 58.928) (end 62.992 57.785) (width 0.254) (layer F.Cu) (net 8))
 (segment (start 64.77 59.483) (end 64.69 59.483) (width 0.254) (layer B.Cu) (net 8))
 (segment (start 64.69 59.483) (end 62.992 57.785) (width 0.254) (layer B.Cu) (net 8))
 (via (at 62.992 57.785) (size 0.6858) (drill 0.3302) (layers F.Cu B.Cu) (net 8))
 (segment (start 62.992 57.785) (end 64.167 56.61) (width 0.254) (layer F.Cu) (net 8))
 (segment (start 64.167 56.61) (end 64.77 56.61) (width 0.254) (layer F.Cu) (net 8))
 (segment (start 80.77 54.61) (end 78.6638 54.61) (width 0.25) (layer F.Cu) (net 21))
 (segment (start 62.0014 50.165) (end 60.325 50.165) (width 0.25) (layer B.Cu) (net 21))
 (segment (start 61.976 53.086) (end 62.0014 50.165) (width 0.25) (layer B.Cu) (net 21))
 (segment (start 66.802 53.086) (end 61.976 53.086) (width 0.25) (layer B.Cu) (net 21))
 (segment (start 68.072 54.229) (end 66.802 53.086) (width 0.25) (layer B.Cu) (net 21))
 (via (at 68.072 54.229) (size 0.6858) (drill 0.3302) (layers F.Cu B.Cu) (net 21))
 (segment (start 78.232 54.229) (end 68.072 54.229) (width 0.25) (layer F.Cu) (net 21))
 (segment (start 78.6638 54.61) (end 78.232 54.229) (width 0.25) (layer F.Cu) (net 21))
 (segment (start 61.594052 53.543815) (end 61.163815 53.543815) (width 0.254) (layer B.Cu) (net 20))
 (segment (start 61.163815 53.543815) (end 60.325 52.705) (width 0.254) (layer B.Cu) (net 20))
 (segment (start 67.437 54.737) (end 66.548 53.594) (width 0.254) (layer B.Cu) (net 20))
 (segment (start 67.8942 55.3212) (end 67.437 54.737) (width 0.254) (layer B.Cu) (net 20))
 (via (at 67.8942 55.3212) (size 0.6858) (drill 0.3302) (layers F.Cu B.Cu) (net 20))
 (segment (start 68.072 55.499) (end 67.8942 55.3212) (width 0.254) (layer F.Cu) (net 20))
 (segment (start 76.706031 55.3667) (end 68.072 55.499) (width 0.254) (layer F.Cu) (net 20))
 (segment (start 66.548 53.594) (end 65.659 53.594) (width 0.254) (layer B.Cu) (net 20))
 (segment (start 79.6478 56.61) (end 76.706031 55.3667) (width 0.254) (layer F.Cu) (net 20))
 (segment (start 65.659 53.594) (end 61.594052 53.543815) (width 0.254) (layer B.Cu) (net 20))
 (segment (start 61.594052 53.543815) (end 61.5442 53.5432) (width 0.254) (layer B.Cu) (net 20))
 (segment (start 61.5442 53.5432) (end 61.468 53.467) (width 0.254) (layer B.Cu) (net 20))
 (segment (start 80.77 56.61) (end 79.6478 56.61) (width 0.254) (layer F.Cu) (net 20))
 (segment (start 60.452 65.913) (end 60.452 65.151) (width 0.254) (layer F.Cu) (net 10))
 (segment (start 60.452 65.151) (end 62.993 62.61) (width 0.254) (layer F.Cu) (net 10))
 (segment (start 62.993 62.61) (end 64.77 62.61) (width 0.254) (layer F.Cu) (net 10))
 (segment (start 64.77 62.61) (end 63.9816 62.61) (width 0.25) (layer F.Cu) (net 10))
 (segment (start 67.818 58.213) (end 66.849 58.213) (width 0.254) (layer B.Cu) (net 9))
 (segment (start 66.294 57.658) (end 65.342 58.61) (width 0.254) (layer F.Cu) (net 9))
 (via (at 66.294 57.658) (size 0.6858) (drill 0.3302) (layers F.Cu B.Cu) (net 9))
 (segment (start 66.849 58.213) (end 66.294 57.658) (width 0.254) (layer B.Cu) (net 9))
 (segment (start 65.342 58.61) (end 64.77 58.61) (width 0.254) (layer F.Cu) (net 9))
 (segment (start 64.77 58.61) (end 65.723 58.61) (width 0.25) (layer F.Cu) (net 9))
 (segment (start 64.77 62.183) (end 64.436 62.183) (width 0.254) (layer B.Cu) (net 11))
 (segment (start 64.436 62.183) (end 62.992 63.627) (width 0.254) (layer B.Cu) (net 11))
 (via (at 62.992 63.627) (size 0.6858) (drill 0.3302) (layers F.Cu B.Cu) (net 11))
 (segment (start 62.992 63.627) (end 63.975 64.61) (width 0.254) (layer F.Cu) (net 11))
 (segment (start 63.975 64.61) (end 64.77 64.61) (width 0.254) (layer F.Cu) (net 11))
 (segment (start 64.77 64.61) (end 63.9902 64.61) (width 0.25) (layer F.Cu) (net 11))
 (segment (start 62.738 66.675) (end 62.611 66.548) (width 0.25) (layer F.Cu) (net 12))
 (segment (start 62.738 70.739) (end 67.945 73.545) (width 0.25) (layer B.Cu) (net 12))
 (segment (start 62.738 67.945) (end 62.738 70.739) (width 0.25) (layer B.Cu) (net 12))
 (segment (start 62.738 66.675) (end 62.738 67.945) (width 0.25) (layer B.Cu) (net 12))
 (via (at 62.738 66.675) (size 0.6858) (drill 0.3302) (layers F.Cu B.Cu) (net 12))
 (segment (start 62.611 66.548) (end 62.738 66.675) (width 0.25) (layer F.Cu) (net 12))
 (segment (start 64.77 66.61) (end 64.77 66.675) (width 0.25) (layer F.Cu) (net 12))
 (segment (start 64.7304 66.7146) (end 62.738 66.675) (width 0.25) (layer F.Cu) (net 12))
 (segment (start 62.738 66.675) (end 62.738 66.7004) (width 0.25) (layer F.Cu) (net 12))
 (segment (start 64.77 66.675) (end 64.7304 66.7146) (width 0.25) (layer F.Cu) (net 12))
 (segment (start 75.358 68.453) (end 75.358 68.025) (width 0.254) (layer B.Cu) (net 15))
 (segment (start 75.358 68.025) (end 76.454 66.929) (width 0.254) (layer B.Cu) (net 15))
 (segment (start 76.454 66.929) (end 78.486 66.929) (width 0.254) (layer B.Cu) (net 15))
 (via (at 78.486 66.929) (size 0.6858) (drill 0.3302) (layers F.Cu B.Cu) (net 15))
 (segment (start 78.486 66.929) (end 78.805 66.61) (width 0.254) (layer F.Cu) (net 15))
 (segment (start 78.805 66.61) (end 80.77 66.61) (width 0.254) (layer F.Cu) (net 15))
 (segment (start 80.772 60.913) (end 81.36 60.913) (width 0.254) (layer B.Cu) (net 16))
 (segment (start 81.36 60.913) (end 83.566 63.119) (width 0.254) (layer B.Cu) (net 16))
 (segment (start 83.566 63.119) (end 83.566 63.627) (width 0.254) (layer B.Cu) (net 16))
 (segment (start 83.566 63.627) (end 82.804 64.389) (width 0.254) (layer B.Cu) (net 16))
 (via (at 82.804 64.389) (size 0.6858) (drill 0.3302) (layers F.Cu B.Cu) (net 16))
 (segment (start 82.804 64.389) (end 82.583 64.61) (width 0.254) (layer F.Cu) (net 16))
 (segment (start 82.583 64.61) (end 80.77 64.61) (width 0.254) (layer F.Cu) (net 16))
 (segment (start 78.867 41.803) (end 80.74374 41.803) (width 0.254) (layer B.Cu) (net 25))
 (segment (start 80.74374 41.803) (end 82.55 43.60926) (width 0.254) (layer B.Cu) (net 25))
 (segment (start 76.073 41.783) (end 78.847 41.783) (width 0.254) (layer B.Cu) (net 25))
 (segment (start 78.847 41.783) (end 78.867 41.803) (width 0.254) (layer B.Cu) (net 25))
 (segment (start 72.644 41.783) (end 76.073 41.783) (width 0.254) (layer B.Cu) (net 25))
 (segment (start 75.926 41.783) (end 75.946 41.803) (width 0.254) (layer B.Cu) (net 25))
 (via (at 78.486 53.213) (size 0.6858) (drill 0.3302) (layers F.Cu B.Cu) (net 25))
 (segment (start 78.486 53.213) (end 78.232 52.959) (width 0.254) (layer B.Cu) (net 25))
 (segment (start 78.232 52.959) (end 72.644 52.959) (width 0.254) (layer B.Cu) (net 25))
 (segment (start 72.644 52.959) (end 72.644 54.67096) (width 0.254) (layer B.Cu) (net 25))
 (segment (start 82.55 43.60926) (end 82.55 45.847) (width 0.254) (layer B.Cu) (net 25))
 (segment (start 81.788 53.213) (end 78.486 53.213) (width 0.254) (layer F.Cu) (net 25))
 (segment (start 82.55 52.451) (end 81.788 53.213) (width 0.254) (layer F.Cu) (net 25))
 (segment (start 82.55 46.863) (end 82.55 52.451) (width 0.254) (layer F.Cu) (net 25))
 (segment (start 83.058 46.355) (end 82.55 46.863) (width 0.254) (layer F.Cu) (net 25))
 (via (at 83.058 46.355) (size 0.6858) (drill 0.3302) (layers F.Cu B.Cu) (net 25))
 (segment (start 82.55 45.847) (end 83.058 46.355) (width 0.254) (layer B.Cu) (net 25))
 (segment (start 82.296 73.025) (end 82.296 65.579) (width 0.254) (layer B.Cu) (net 17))
 (segment (start 82.296 65.579) (end 80.772 64.055) (width 0.254) (layer B.Cu) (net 17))
 (segment (start 80.77 62.61) (end 81.787 62.61) (width 0.254) (layer F.Cu) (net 17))
 (segment (start 81.787 62.61) (end 82.55 63.373) (width 0.254) (layer F.Cu) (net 17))
 (segment (start 81.868 64.055) (end 80.772 64.055) (width 0.254) (layer B.Cu) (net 17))
 (segment (start 82.55 63.373) (end 81.868 64.055) (width 0.254) (layer B.Cu) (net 17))
 (via (at 82.55 63.373) (size 0.6858) (drill 0.3302) (layers F.Cu B.Cu) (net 17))
 (segment (start 80.0598 62.61) (end 80.77 62.61) (width 0.25) (layer F.Cu) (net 17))
 (segment (start 64.77 54.61) (end 65.278 54.61) (width 0.25) (layer F.Cu) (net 7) (status 80000))
 (segment (start 64.77 53.0606) (end 64.77 53.086) (width 0.25) (layer F.Cu) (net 7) (status 80000))
 (segment (start 64.77 53.086) (end 64.77 54.61) (width 0.25) (layer F.Cu) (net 7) (status 80000))
 (segment (start 64.77 60.61) (end 65.6646 60.61) (width 0.25) (layer F.Cu) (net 7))
 (segment (start 60.452 68.453) (end 60.452 69.469) (width 0.254) (layer B.Cu) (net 24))
 (segment (start 60.452 69.469) (end 62.738 71.755) (width 0.254) (layer B.Cu) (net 24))
 (segment (start 62.738 71.755) (end 63.246 71.755) (width 0.254) (layer B.Cu) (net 24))
 (segment (start 63.246 71.755) (end 67.136 75.645) (width 0.254) (layer B.Cu) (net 24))
 (segment (start 67.136 75.645) (end 67.945 75.645) (width 0.254) (layer B.Cu) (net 24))
 (segment (start 72.39 76.835) (end 69.135 76.835) (width 0.254) (layer B.Cu) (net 24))
 (segment (start 69.135 76.835) (end 67.945 75.645) (width 0.254) (layer B.Cu) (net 24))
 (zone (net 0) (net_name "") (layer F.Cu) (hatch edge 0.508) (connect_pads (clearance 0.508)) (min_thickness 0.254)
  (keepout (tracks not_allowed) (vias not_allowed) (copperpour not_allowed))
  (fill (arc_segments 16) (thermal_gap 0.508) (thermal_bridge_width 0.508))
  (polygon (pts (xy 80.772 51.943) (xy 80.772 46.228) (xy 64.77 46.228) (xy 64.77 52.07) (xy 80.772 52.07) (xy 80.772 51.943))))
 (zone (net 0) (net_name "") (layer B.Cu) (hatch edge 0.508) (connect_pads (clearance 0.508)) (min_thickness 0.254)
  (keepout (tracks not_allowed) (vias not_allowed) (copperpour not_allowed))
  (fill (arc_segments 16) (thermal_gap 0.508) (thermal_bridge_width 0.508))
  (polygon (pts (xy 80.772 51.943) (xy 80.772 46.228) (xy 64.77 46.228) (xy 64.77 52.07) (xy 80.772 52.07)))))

